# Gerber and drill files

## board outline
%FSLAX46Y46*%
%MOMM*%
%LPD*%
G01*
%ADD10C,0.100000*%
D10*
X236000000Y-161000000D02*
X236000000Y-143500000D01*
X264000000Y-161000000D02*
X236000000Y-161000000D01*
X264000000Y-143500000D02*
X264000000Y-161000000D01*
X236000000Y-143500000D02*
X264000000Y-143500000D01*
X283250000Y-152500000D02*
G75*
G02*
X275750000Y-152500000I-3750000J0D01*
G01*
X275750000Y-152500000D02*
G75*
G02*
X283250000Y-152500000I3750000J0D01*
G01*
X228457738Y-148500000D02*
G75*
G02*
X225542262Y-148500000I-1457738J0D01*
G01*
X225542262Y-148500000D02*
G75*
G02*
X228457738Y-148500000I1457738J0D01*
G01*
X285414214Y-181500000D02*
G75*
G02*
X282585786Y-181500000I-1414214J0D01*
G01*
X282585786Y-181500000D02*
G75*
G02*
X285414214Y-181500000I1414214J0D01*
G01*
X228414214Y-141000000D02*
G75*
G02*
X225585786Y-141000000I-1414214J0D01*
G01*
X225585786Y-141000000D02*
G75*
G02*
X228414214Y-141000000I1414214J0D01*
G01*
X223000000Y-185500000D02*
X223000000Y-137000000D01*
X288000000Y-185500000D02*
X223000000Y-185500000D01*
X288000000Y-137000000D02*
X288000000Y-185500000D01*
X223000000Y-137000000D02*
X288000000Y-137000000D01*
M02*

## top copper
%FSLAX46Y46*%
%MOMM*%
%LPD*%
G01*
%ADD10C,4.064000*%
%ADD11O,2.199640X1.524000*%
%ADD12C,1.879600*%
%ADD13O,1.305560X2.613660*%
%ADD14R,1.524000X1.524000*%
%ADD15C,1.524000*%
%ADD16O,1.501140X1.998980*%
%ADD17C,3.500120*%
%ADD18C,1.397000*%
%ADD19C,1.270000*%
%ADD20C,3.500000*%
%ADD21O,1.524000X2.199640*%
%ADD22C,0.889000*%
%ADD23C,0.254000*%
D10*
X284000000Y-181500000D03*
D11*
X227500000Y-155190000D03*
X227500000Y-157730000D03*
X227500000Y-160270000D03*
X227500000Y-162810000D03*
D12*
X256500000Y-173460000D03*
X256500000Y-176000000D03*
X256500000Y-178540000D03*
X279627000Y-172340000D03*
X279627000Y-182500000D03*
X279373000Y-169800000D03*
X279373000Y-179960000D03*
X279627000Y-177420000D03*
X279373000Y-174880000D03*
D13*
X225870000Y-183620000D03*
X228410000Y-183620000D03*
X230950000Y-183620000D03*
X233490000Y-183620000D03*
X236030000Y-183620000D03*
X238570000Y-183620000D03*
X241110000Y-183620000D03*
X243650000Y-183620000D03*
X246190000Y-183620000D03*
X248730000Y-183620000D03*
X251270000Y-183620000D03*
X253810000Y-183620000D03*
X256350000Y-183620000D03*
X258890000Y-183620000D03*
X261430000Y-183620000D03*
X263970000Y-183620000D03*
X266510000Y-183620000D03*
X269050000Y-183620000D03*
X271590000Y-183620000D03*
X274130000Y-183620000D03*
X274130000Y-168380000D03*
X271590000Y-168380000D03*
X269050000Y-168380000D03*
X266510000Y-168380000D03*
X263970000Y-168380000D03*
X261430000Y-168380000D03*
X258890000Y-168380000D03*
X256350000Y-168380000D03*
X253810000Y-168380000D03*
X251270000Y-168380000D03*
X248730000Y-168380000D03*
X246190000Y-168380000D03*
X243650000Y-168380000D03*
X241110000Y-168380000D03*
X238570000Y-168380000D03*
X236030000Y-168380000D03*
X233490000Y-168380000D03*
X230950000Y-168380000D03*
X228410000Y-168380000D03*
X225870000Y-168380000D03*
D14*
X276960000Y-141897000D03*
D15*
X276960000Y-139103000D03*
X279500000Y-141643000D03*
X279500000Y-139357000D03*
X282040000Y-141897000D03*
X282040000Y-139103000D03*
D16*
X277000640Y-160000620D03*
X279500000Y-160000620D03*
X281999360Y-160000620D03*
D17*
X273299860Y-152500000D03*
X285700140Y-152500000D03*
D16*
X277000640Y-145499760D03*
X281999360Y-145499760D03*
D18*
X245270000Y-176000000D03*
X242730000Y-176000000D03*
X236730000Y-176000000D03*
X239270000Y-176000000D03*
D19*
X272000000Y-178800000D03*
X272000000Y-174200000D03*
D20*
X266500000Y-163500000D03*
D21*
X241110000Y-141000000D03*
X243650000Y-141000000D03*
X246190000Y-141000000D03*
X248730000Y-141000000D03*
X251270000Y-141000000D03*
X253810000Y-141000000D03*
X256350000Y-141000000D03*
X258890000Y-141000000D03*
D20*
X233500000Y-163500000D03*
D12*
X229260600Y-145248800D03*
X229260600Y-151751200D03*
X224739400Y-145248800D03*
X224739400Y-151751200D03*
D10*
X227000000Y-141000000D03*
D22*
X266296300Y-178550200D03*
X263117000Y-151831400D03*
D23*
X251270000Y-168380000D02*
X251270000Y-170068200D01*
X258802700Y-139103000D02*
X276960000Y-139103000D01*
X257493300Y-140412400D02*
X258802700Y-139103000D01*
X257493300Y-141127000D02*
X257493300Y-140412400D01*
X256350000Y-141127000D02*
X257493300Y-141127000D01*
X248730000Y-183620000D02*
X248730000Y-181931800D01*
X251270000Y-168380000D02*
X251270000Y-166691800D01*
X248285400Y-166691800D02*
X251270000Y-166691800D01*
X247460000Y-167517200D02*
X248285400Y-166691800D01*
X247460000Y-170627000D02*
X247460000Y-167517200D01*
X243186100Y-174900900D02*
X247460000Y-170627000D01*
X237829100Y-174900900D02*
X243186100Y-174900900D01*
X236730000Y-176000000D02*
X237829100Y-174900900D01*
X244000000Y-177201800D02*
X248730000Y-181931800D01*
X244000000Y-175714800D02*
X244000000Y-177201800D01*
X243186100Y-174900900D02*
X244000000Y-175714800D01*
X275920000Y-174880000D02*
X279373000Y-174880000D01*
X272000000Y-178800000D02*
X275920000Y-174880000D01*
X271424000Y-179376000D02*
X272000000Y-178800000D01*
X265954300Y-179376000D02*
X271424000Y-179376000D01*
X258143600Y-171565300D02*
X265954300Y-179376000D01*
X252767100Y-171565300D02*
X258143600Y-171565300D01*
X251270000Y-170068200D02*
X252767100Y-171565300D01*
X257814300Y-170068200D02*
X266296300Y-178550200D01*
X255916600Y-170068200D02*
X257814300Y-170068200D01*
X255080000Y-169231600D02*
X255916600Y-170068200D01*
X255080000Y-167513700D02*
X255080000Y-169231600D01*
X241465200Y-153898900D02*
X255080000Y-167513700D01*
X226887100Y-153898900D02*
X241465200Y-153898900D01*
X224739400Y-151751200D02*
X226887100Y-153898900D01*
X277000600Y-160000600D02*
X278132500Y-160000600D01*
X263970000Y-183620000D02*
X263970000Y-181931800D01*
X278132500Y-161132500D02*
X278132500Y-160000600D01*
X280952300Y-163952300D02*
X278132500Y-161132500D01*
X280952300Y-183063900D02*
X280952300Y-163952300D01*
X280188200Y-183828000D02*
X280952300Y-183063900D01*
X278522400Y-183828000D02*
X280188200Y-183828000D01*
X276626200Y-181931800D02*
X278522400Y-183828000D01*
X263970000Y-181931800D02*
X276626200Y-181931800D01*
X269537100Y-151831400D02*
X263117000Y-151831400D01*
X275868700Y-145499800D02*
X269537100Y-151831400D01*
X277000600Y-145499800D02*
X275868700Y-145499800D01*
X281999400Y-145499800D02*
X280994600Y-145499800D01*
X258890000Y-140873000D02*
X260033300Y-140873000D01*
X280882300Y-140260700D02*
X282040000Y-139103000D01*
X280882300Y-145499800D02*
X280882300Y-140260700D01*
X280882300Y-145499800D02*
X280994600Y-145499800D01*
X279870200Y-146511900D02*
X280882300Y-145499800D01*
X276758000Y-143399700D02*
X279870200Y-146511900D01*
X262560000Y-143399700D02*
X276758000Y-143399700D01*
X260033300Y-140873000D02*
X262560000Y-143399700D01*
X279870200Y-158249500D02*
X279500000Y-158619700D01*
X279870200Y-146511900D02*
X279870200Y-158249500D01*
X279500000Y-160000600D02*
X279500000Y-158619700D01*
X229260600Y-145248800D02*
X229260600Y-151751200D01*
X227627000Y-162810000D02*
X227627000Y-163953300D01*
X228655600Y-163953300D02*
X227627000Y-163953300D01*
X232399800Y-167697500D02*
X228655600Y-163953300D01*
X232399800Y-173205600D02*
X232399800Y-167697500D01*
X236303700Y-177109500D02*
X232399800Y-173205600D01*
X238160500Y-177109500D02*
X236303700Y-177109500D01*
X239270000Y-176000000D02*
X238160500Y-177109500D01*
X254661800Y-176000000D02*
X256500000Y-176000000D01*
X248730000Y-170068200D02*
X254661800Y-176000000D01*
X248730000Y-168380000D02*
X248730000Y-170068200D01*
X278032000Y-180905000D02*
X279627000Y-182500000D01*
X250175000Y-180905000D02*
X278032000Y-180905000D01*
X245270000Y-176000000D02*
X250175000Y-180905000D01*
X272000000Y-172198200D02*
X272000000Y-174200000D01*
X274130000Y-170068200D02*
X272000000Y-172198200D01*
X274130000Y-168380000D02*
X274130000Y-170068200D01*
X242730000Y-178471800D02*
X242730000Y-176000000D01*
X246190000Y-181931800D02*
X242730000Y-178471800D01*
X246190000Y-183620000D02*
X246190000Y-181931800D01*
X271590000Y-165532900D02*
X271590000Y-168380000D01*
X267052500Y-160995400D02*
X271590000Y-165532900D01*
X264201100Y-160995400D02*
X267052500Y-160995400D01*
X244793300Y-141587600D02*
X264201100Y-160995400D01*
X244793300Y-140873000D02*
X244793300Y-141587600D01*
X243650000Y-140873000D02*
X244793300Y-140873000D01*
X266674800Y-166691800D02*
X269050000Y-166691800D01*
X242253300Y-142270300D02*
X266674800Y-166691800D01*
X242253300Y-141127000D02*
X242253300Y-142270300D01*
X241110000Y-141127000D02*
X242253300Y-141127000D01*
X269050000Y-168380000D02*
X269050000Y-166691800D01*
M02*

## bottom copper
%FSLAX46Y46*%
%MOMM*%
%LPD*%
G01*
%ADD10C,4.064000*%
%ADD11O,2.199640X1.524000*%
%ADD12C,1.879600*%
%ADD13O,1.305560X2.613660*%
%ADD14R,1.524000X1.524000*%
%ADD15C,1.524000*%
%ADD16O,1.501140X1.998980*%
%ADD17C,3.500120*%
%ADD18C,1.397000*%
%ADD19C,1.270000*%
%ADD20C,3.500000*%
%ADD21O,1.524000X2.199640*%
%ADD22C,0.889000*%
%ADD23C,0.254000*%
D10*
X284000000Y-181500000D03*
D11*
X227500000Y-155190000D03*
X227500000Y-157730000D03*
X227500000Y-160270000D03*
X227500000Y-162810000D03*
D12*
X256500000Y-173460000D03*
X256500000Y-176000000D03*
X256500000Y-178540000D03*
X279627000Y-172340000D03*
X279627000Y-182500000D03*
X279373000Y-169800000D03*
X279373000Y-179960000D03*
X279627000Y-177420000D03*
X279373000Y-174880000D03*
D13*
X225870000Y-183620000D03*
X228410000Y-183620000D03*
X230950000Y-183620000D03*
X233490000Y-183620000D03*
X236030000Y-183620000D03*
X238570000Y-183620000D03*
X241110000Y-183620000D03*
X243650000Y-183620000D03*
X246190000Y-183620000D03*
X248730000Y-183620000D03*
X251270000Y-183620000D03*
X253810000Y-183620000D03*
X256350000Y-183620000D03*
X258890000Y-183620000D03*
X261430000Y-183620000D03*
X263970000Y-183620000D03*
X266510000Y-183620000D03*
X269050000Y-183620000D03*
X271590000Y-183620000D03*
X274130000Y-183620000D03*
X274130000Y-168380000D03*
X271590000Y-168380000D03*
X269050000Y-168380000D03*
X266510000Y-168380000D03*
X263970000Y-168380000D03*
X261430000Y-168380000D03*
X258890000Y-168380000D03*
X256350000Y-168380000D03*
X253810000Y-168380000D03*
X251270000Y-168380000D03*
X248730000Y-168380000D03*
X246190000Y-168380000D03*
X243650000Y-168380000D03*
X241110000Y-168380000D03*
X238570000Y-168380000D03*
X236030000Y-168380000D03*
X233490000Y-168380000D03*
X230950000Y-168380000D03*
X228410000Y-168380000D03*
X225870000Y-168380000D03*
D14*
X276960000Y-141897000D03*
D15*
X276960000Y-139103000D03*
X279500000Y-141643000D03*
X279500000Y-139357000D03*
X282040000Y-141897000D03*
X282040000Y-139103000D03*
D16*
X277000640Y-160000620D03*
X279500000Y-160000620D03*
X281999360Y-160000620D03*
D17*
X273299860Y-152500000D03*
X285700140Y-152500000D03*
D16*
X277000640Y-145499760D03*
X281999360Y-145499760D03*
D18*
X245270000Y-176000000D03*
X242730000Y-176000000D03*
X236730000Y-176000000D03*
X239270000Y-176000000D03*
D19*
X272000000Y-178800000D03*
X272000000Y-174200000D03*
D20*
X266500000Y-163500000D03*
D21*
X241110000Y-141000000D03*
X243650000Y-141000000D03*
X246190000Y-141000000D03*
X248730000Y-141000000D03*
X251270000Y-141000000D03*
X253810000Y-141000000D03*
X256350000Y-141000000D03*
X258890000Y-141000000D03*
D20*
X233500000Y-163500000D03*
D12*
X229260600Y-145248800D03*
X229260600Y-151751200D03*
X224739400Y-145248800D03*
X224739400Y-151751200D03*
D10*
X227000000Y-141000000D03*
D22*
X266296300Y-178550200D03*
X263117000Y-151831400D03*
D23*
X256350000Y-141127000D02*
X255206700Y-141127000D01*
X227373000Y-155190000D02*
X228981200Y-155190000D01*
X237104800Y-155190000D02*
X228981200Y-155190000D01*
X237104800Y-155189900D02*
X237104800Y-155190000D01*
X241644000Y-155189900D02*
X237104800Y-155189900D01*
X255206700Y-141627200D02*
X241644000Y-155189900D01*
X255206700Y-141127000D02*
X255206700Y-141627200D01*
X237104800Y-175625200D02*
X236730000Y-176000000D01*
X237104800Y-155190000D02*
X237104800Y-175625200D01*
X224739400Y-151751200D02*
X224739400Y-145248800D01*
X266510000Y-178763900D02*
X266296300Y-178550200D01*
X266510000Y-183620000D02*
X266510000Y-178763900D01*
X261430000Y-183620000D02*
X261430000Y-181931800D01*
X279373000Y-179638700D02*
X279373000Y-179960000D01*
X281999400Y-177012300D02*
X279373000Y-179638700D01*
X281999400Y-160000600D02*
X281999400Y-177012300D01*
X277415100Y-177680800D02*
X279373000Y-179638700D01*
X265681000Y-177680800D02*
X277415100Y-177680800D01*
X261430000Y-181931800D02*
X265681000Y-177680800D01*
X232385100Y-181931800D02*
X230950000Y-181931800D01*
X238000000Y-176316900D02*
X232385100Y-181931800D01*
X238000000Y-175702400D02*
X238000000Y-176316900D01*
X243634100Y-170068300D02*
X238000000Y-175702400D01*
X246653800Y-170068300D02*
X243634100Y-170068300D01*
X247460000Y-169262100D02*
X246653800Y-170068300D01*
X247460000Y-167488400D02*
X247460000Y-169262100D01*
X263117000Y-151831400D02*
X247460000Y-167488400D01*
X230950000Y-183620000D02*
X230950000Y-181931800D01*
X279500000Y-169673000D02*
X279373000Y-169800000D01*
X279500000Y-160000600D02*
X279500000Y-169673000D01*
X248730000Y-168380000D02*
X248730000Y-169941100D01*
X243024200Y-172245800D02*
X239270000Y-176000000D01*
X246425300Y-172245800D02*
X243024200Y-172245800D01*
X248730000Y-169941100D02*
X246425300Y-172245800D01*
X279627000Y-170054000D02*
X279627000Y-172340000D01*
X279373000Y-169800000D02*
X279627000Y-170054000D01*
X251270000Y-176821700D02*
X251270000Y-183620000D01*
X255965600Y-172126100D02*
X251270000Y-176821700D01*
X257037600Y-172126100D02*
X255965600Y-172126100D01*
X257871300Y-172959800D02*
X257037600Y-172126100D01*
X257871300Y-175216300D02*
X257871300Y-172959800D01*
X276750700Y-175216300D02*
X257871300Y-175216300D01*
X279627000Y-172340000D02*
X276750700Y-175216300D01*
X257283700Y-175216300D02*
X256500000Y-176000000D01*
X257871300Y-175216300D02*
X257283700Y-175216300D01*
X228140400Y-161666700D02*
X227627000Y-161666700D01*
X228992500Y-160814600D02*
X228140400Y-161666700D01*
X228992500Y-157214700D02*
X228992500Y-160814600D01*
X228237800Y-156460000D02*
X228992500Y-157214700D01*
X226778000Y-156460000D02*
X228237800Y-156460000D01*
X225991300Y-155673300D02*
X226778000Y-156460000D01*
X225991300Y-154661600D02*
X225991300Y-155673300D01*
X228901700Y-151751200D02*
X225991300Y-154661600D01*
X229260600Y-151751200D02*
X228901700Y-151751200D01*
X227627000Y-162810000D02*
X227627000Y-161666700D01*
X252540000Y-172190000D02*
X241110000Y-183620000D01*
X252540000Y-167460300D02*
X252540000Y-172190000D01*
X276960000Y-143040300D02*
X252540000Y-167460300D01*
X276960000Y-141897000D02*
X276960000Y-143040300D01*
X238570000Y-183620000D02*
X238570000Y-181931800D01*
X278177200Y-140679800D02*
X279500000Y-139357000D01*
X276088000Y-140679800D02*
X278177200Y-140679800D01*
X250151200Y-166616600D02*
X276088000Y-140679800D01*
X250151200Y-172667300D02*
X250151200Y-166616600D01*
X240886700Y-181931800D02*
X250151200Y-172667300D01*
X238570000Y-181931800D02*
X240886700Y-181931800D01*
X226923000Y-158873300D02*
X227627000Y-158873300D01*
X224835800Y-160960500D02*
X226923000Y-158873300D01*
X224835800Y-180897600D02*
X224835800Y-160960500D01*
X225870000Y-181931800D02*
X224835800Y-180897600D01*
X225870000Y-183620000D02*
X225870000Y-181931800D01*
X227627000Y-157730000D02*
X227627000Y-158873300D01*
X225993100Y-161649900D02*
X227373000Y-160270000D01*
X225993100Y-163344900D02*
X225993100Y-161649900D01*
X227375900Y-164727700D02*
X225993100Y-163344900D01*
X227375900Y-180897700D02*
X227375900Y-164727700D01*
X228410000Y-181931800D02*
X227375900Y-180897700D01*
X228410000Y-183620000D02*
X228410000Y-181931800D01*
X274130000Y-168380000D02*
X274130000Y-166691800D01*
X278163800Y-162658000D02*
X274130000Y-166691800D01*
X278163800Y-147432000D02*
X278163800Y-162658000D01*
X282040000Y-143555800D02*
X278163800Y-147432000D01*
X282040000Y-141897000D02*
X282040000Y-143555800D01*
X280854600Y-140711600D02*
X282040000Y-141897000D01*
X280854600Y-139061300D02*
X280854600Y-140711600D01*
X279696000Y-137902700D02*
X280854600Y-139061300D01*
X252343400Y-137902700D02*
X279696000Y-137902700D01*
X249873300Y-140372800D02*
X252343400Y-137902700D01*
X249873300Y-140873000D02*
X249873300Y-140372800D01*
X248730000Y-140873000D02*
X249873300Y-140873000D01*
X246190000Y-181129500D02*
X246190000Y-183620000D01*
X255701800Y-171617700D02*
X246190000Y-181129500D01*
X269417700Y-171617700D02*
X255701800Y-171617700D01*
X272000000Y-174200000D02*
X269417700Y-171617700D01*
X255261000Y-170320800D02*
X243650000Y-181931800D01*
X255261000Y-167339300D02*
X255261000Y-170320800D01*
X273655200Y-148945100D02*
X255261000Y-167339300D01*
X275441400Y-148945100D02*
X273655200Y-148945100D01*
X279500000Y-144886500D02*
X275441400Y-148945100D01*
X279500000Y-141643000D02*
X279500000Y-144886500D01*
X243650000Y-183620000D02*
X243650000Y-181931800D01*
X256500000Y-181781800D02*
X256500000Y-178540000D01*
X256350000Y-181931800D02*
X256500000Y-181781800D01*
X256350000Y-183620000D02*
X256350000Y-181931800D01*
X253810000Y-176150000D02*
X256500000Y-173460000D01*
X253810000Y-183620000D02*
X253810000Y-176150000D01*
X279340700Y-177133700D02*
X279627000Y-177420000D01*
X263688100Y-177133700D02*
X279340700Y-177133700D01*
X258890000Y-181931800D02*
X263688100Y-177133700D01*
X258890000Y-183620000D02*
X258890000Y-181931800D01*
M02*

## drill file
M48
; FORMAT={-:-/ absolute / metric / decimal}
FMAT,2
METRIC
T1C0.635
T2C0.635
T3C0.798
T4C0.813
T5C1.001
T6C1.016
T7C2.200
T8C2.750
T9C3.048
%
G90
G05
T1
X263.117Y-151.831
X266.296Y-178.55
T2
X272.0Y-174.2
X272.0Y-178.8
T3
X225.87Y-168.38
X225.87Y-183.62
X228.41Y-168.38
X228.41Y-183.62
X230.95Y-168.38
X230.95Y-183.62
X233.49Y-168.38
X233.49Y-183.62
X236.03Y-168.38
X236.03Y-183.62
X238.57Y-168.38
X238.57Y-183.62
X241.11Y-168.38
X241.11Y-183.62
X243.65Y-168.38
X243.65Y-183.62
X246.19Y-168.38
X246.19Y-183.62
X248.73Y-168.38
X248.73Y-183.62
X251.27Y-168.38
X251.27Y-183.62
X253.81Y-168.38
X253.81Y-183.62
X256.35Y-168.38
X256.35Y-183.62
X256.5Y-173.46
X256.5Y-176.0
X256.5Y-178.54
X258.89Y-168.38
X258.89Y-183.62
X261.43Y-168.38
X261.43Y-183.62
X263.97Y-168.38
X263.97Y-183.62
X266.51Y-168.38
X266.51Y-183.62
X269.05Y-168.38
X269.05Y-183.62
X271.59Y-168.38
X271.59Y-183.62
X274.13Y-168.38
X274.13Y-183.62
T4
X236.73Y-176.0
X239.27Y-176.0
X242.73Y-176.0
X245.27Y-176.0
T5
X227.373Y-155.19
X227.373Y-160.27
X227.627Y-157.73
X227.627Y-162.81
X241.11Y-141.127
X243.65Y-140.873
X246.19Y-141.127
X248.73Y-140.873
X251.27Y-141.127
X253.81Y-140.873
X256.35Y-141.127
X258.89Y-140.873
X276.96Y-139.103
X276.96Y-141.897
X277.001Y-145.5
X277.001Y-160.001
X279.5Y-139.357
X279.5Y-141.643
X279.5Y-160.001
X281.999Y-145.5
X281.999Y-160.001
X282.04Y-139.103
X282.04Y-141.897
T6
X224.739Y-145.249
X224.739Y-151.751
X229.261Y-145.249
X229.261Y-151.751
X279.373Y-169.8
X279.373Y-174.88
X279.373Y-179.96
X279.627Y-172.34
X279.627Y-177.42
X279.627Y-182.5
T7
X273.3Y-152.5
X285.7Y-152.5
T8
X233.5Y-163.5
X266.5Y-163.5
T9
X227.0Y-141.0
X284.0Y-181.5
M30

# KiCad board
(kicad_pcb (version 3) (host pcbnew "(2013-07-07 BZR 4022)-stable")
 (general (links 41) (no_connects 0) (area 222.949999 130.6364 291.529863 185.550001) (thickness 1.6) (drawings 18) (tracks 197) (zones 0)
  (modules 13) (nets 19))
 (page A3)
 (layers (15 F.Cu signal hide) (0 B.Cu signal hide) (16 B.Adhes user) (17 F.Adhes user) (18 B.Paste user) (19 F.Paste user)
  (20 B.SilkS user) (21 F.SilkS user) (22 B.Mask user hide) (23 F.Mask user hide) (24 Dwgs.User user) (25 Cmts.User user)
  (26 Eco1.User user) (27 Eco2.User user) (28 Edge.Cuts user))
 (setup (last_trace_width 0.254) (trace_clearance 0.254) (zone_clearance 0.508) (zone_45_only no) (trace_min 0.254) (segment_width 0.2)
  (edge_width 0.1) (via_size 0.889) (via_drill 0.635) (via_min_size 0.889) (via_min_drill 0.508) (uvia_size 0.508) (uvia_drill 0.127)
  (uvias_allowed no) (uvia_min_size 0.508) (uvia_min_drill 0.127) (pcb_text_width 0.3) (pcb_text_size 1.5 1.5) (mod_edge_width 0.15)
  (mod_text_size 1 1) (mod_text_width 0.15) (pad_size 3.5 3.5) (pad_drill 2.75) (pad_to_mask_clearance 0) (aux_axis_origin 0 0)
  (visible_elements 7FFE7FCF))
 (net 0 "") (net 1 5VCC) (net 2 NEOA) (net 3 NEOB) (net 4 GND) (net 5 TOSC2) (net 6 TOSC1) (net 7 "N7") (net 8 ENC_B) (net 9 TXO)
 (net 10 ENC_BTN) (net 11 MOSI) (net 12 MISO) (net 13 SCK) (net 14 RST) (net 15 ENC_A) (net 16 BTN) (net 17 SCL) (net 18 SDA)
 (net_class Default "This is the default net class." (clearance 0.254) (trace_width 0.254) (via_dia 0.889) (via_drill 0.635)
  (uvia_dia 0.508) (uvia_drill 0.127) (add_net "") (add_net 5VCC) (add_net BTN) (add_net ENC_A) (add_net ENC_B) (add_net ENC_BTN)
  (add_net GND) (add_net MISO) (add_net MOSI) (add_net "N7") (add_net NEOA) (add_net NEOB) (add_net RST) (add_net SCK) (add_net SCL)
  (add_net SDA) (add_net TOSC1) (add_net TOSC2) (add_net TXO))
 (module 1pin (layer F.Cu) (at 284 181.5)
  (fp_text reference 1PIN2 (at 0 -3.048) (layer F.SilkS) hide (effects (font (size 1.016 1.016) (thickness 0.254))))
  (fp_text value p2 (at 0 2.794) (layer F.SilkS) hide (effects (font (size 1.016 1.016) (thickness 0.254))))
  (pad 1 thru_hole circle (at 0 0) (size 4.064 4.064) (drill 3.048) (layers *.Cu *.Mask F.SilkS)))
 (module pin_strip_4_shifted (layer F.Cu) (at 227.5 159 270)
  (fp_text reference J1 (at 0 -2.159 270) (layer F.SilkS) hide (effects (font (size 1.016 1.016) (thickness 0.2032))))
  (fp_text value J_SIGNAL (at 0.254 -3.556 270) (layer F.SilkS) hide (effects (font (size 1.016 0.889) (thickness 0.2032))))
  (pad 1 thru_hole oval (at -3.81 0.127 270) (size 1.524 2.19964) (drill 1.00076 (offset 0 -0.127)) (layers *.Cu *.Mask F.SilkS)
   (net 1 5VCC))
  (pad 2 thru_hole oval (at -1.27 -0.127 270) (size 1.524 2.19964) (drill 1.00076 (offset 0 0.127)) (layers *.Cu *.Mask F.SilkS)
   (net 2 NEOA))
  (pad 3 thru_hole oval (at 1.27 0.127 270) (size 1.524 2.19964) (drill 1.00076 (offset 0 -0.127)) (layers *.Cu *.Mask F.SilkS) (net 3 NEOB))
  (pad 4 thru_hole oval (at 3.81 -0.127 270) (size 1.524 2.19964) (drill 1.00076 (offset 0 0.127)) (layers *.Cu *.Mask F.SilkS) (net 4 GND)))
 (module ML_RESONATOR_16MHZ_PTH (layer F.Cu) (at 256.5 176 270)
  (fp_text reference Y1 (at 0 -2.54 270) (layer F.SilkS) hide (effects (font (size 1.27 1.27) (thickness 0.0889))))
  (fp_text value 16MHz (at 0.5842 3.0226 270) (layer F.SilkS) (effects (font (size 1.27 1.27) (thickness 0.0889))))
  (pad 1 thru_hole circle (at -2.54 0 270) (size 1.8796 1.8796) (drill 0.79756) (layers *.Cu *.Mask F.Paste F.SilkS) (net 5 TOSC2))
  (pad 2 thru_hole circle (at 0 0 270) (size 1.8796 1.8796) (drill 0.79756) (layers *.Cu *.Mask F.Paste F.SilkS) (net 4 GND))
  (pad 3 thru_hole circle (at 2.54 0 270) (size 1.8796 1.8796) (drill 0.79756) (layers *.Cu *.Mask F.Paste F.SilkS) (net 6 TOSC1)))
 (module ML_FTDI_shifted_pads (layer F.Cu) (at 279.5 182.5 90)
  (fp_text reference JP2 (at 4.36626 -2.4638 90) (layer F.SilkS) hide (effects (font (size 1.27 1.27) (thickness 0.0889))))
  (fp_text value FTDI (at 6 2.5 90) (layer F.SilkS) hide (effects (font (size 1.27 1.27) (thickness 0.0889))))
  (pad CTS thru_hole circle (at 10.16 0.127 90) (size 1.8796 1.8796) (drill 1.016) (layers *.Cu *.Mask F.Paste F.SilkS) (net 4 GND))
  (pad DTR thru_hole circle (at 0 0.127 90) (size 1.8796 1.8796) (drill 1.016) (layers *.Cu *.Mask F.Paste F.SilkS) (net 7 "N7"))
  (pad GND thru_hole circle (at 12.7 -0.127 90) (size 1.8796 1.8796) (drill 1.016) (layers *.Cu *.Mask F.Paste F.SilkS) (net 4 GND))
  (pad RXI thru_hole circle (at 2.54 -0.127 90) (size 1.8796 1.8796) (drill 1.016) (layers *.Cu *.Mask F.Paste F.SilkS) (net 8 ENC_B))
  (pad TXO thru_hole circle (at 5.08 0.127 90) (size 1.8796 1.8796) (drill 1.016) (layers *.Cu *.Mask F.Paste F.SilkS) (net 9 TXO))
  (pad VCC thru_hole circle (at 7.62 -0.127 90) (size 1.8796 1.8796) (drill 1.016) (layers *.Cu *.Mask F.Paste F.SilkS) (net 1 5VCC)))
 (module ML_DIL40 (layer F.Cu) (at 250 176)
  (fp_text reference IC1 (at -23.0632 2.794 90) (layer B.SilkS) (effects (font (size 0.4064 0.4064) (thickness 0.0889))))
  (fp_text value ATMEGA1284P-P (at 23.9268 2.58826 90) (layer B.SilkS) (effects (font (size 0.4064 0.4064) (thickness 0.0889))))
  (pad 1 thru_hole oval (at -24.13 7.62) (size 1.30556 2.61366) (drill 0.79756) (layers *.Cu *.Mask F.Paste F.SilkS) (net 2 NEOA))
  (pad 2 thru_hole oval (at -21.59 7.62) (size 1.30556 2.61366) (drill 0.79756) (layers *.Cu *.Mask F.Paste F.SilkS) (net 3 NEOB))
  (pad 3 thru_hole oval (at -19.05 7.62) (size 1.30556 2.61366) (drill 0.79756) (layers *.Cu *.Mask F.Paste F.SilkS) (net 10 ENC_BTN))
  (pad 4 thru_hole oval (at -16.51 7.62) (size 1.30556 2.61366) (drill 0.79756) (layers *.Cu *.Mask F.Paste F.SilkS))
  (pad 5 thru_hole oval (at -13.97 7.62) (size 1.30556 2.61366) (drill 0.79756) (layers *.Cu *.Mask F.Paste F.SilkS))
  (pad 6 thru_hole oval (at -11.43 7.62) (size 1.30556 2.61366) (drill 0.79756) (layers *.Cu *.Mask F.Paste F.SilkS) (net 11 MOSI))
  (pad 7 thru_hole oval (at -8.89 7.62) (size 1.30556 2.61366) (drill 0.79756) (layers *.Cu *.Mask F.Paste F.SilkS) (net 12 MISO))
  (pad 8 thru_hole oval (at -6.35 7.62) (size 1.30556 2.61366) (drill 0.79756) (layers *.Cu *.Mask F.Paste F.SilkS) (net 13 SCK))
  (pad 9 thru_hole oval (at -3.81 7.62) (size 1.30556 2.61366) (drill 0.79756) (layers *.Cu *.Mask F.Paste F.SilkS) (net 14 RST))
  (pad 10 thru_hole oval (at -1.27 7.62) (size 1.30556 2.61366) (drill 0.79756) (layers *.Cu *.Mask F.Paste F.SilkS) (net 1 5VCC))
  (pad 11 thru_hole oval (at 1.27 7.62) (size 1.30556 2.61366) (drill 0.79756) (layers *.Cu *.Mask F.Paste F.SilkS) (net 4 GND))
  (pad 12 thru_hole oval (at 3.81 7.62) (size 1.30556 2.61366) (drill 0.79756) (layers *.Cu *.Mask F.Paste F.SilkS) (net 5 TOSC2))
  (pad 13 thru_hole oval (at 6.35 7.62) (size 1.30556 2.61366) (drill 0.79756) (layers *.Cu *.Mask F.Paste F.SilkS) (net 6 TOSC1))
  (pad 14 thru_hole oval (at 8.89 7.62) (size 1.30556 2.61366) (drill 0.79756) (layers *.Cu *.Mask F.Paste F.SilkS) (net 9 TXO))
  (pad 15 thru_hole oval (at 11.43 7.62) (size 1.30556 2.61366) (drill 0.79756) (layers *.Cu *.Mask F.Paste F.SilkS) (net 8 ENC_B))
  (pad 16 thru_hole oval (at 13.97 7.62) (size 1.30556 2.61366) (drill 0.79756) (layers *.Cu *.Mask F.Paste F.SilkS) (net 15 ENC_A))
  (pad 17 thru_hole oval (at 16.51 7.62) (size 1.30556 2.61366) (drill 0.79756) (layers *.Cu *.Mask F.Paste F.SilkS) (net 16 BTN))
  (pad 18 thru_hole oval (at 19.05 7.62) (size 1.30556 2.61366) (drill 0.79756) (layers *.Cu *.Mask F.Paste F.SilkS))
  (pad 19 thru_hole oval (at 21.59 7.62) (size 1.30556 2.61366) (drill 0.79756) (layers *.Cu *.Mask F.Paste F.SilkS))
  (pad 20 thru_hole oval (at 24.13 7.62) (size 1.30556 2.61366) (drill 0.79756) (layers *.Cu *.Mask F.Paste F.SilkS))
  (pad 21 thru_hole oval (at 24.13 -7.62) (size 1.30556 2.61366) (drill 0.79756) (layers *.Cu *.Mask F.Paste F.SilkS) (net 14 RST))
  (pad 22 thru_hole oval (at 21.59 -7.62) (size 1.30556 2.61366) (drill 0.79756) (layers *.Cu *.Mask F.Paste F.SilkS) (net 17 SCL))
  (pad 23 thru_hole oval (at 19.05 -7.62) (size 1.30556 2.61366) (drill 0.79756) (layers *.Cu *.Mask F.Paste F.SilkS) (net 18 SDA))
  (pad 24 thru_hole oval (at 16.51 -7.62) (size 1.30556 2.61366) (drill 0.79756) (layers *.Cu *.Mask F.Paste F.SilkS))
  (pad 25 thru_hole oval (at 13.97 -7.62) (size 1.30556 2.61366) (drill 0.79756) (layers *.Cu *.Mask F.Paste F.SilkS))
  (pad 26 thru_hole oval (at 11.43 -7.62) (size 1.30556 2.61366) (drill 0.79756) (layers *.Cu *.Mask F.Paste F.SilkS))
  (pad 27 thru_hole oval (at 8.89 -7.62) (size 1.30556 2.61366) (drill 0.79756) (layers *.Cu *.Mask F.Paste F.SilkS))
  (pad 28 thru_hole oval (at 6.35 -7.62) (size 1.30556 2.61366) (drill 0.79756) (layers *.Cu *.Mask F.Paste F.SilkS))
  (pad 29 thru_hole oval (at 3.81 -7.62) (size 1.30556 2.61366) (drill 0.79756) (layers *.Cu *.Mask F.Paste F.SilkS))
  (pad 30 thru_hole oval (at 1.27 -7.62) (size 1.30556 2.61366) (drill 0.79756) (layers *.Cu *.Mask F.Paste F.SilkS) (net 1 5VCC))
  (pad 31 thru_hole oval (at -1.27 -7.62) (size 1.30556 2.61366) (drill 0.79756) (layers *.Cu *.Mask F.Paste F.SilkS) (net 4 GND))
  (pad 32 thru_hole oval (at -3.81 -7.62) (size 1.30556 2.61366) (drill 0.79756) (layers *.Cu *.Mask F.Paste F.SilkS))
  (pad 33 thru_hole oval (at -6.35 -7.62) (size 1.30556 2.61366) (drill 0.79756) (layers *.Cu *.Mask F.Paste F.SilkS))
  (pad 34 thru_hole oval (at -8.89 -7.62) (size 1.30556 2.61366) (drill 0.79756) (layers *.Cu *.Mask F.Paste F.SilkS))
  (pad 35 thru_hole oval (at -11.43 -7.62) (size 1.30556 2.61366) (drill 0.79756) (layers *.Cu *.Mask F.Paste F.SilkS))
  (pad 36 thru_hole oval (at -13.97 -7.62) (size 1.30556 2.61366) (drill 0.79756) (layers *.Cu *.Mask F.Paste F.SilkS))
  (pad 37 thru_hole oval (at -16.51 -7.62) (size 1.30556 2.61366) (drill 0.79756) (layers *.Cu *.Mask F.Paste F.SilkS))
  (pad 38 thru_hole oval (at -19.05 -7.62) (size 1.30556 2.61366) (drill 0.79756) (layers *.Cu *.Mask F.Paste F.SilkS))
  (pad 39 thru_hole oval (at -21.59 -7.62) (size 1.30556 2.61366) (drill 0.79756) (layers *.Cu *.Mask F.Paste F.SilkS))
  (pad 40 thru_hole oval (at -24.13 -7.62) (size 1.30556 2.61366) (drill 0.79756) (layers *.Cu *.Mask F.Paste F.SilkS)))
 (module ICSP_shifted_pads (layer F.Cu) (at 279.5 140.5)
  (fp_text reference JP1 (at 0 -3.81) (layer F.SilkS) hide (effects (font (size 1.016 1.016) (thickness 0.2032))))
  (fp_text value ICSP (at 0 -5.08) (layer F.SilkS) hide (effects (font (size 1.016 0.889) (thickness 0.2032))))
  (pad 1 thru_hole rect (at -2.54 1.397) (size 1.524 1.524) (drill 1.00076) (layers *.Cu *.Mask F.SilkS) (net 12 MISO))
  (pad 2 thru_hole circle (at -2.54 -1.397) (size 1.524 1.524) (drill 1.00076) (layers *.Cu *.Mask F.SilkS) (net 1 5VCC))
  (pad 3 thru_hole circle (at 0 1.143) (size 1.524 1.524) (drill 1.00076) (layers *.Cu *.Mask F.SilkS) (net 13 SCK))
  (pad 4 thru_hole circle (at 0 -1.143) (size 1.524 1.524) (drill 1.00076) (layers *.Cu *.Mask F.SilkS) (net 11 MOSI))
  (pad 5 thru_hole circle (at 2.54 1.397) (size 1.524 1.524) (drill 1.00076) (layers *.Cu *.Mask F.SilkS) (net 14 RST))
  (pad 6 thru_hole circle (at 2.54 -1.397) (size 1.524 1.524) (drill 1.00076) (layers *.Cu *.Mask F.SilkS) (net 4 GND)))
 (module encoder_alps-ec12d (layer F.Cu) (at 279.5 152.5) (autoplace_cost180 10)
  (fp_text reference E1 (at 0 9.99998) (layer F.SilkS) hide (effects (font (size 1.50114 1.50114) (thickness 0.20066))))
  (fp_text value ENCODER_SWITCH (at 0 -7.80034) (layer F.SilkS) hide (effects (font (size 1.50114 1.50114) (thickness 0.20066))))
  (pad 1 thru_hole oval (at -2.49936 7.50062) (size 1.50114 1.99898) (drill 1.00076) (layers *.Cu *.Mask F.SilkS) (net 15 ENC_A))
  (pad 2 thru_hole oval (at 0 7.50062) (size 1.50114 1.99898) (drill 1.00076) (layers *.Cu *.Mask F.SilkS) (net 4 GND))
  (pad 3 thru_hole oval (at 2.49936 7.50062) (size 1.50114 1.99898) (drill 1.00076) (layers *.Cu *.Mask F.SilkS) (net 8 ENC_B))
  (pad "" thru_hole circle (at -6.20014 0) (size 3.50012 3.50012) (drill 2.19964) (layers *.Cu *.Mask F.SilkS))
  (pad "" thru_hole circle (at 6.20014 0) (size 3.50012 3.50012) (drill 2.19964) (layers *.Cu *.Mask F.SilkS))
  (pad 5 thru_hole oval (at -2.49936 -7.00024) (size 1.50114 1.99898) (drill 1.00076) (layers *.Cu *.Mask F.SilkS) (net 10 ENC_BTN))
  (pad 4 thru_hole oval (at 2.49936 -7.00024) (size 1.50114 1.99898) (drill 1.00076) (layers *.Cu *.Mask F.SilkS) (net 4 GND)))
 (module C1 (layer F.Cu) (at 244 176 180)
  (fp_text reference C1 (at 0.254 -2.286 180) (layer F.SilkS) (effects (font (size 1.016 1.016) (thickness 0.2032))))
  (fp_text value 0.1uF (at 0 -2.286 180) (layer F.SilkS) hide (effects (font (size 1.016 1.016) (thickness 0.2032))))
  (pad 1 thru_hole circle (at -1.27 0 180) (size 1.397 1.397) (drill 0.8128) (layers *.Cu *.Mask F.SilkS) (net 7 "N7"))
  (pad 2 thru_hole circle (at 1.27 0 180) (size 1.397 1.397) (drill 0.8128) (layers *.Cu *.Mask F.SilkS) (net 14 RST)))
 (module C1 (layer F.Cu) (at 238 176)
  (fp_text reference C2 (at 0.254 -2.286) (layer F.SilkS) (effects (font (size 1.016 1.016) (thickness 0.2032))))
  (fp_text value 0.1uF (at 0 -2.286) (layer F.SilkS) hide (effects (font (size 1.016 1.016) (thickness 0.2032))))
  (pad 1 thru_hole circle (at -1.27 0) (size 1.397 1.397) (drill 0.8128) (layers *.Cu *.Mask F.SilkS) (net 1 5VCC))
  (pad 2 thru_hole circle (at 1.27 0) (size 1.397 1.397) (drill 0.8128) (layers *.Cu *.Mask F.SilkS) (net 4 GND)))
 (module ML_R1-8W (layer F.Cu) (at 272 176.5 90)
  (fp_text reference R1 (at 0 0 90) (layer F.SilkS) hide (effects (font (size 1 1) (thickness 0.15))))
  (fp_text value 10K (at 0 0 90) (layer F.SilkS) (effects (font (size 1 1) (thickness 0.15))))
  (pad 1 thru_hole circle (at -2.3 0 90) (size 1.27 1.27) (drill 0.635) (layers *.Cu *.Mask F.SilkS) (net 1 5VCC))
  (pad 2 thru_hole circle (at 2.3 0 90) (size 1.27 1.27) (drill 0.635) (layers *.Cu *.Mask F.SilkS) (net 14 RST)))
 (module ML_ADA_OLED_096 (layer F.Cu) (at 250 141)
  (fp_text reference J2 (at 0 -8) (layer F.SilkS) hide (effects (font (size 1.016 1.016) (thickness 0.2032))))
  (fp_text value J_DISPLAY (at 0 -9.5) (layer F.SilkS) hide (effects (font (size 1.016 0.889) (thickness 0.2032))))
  (pad 9 thru_hole circle (at 16.5 22.5) (size 3.5 3.5) (drill 2.75) (layers *.Cu *.Mask F.SilkS))
  (pad 1 thru_hole oval (at -8.89 0.127) (size 1.524 2.19964) (drill 1.00076 (offset 0 -0.127)) (layers *.Cu *.Mask F.SilkS) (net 18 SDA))
  (pad 2 thru_hole oval (at -6.35 -0.127) (size 1.524 2.19964) (drill 1.00076 (offset 0 0.127)) (layers *.Cu *.Mask F.SilkS) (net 17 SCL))
  (pad 3 thru_hole oval (at -3.81 0.127) (size 1.524 2.19964) (drill 1.00076 (offset 0 -0.127)) (layers *.Cu *.Mask F.SilkS))
  (pad 4 thru_hole oval (at -1.27 -0.127) (size 1.524 2.19964) (drill 1.00076 (offset 0 0.127)) (layers *.Cu *.Mask F.SilkS) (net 14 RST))
  (pad 5 thru_hole oval (at 1.27 0.127) (size 1.524 2.19964) (drill 1.00076 (offset 0 -0.127)) (layers *.Cu *.Mask F.SilkS))
  (pad 6 thru_hole oval (at 3.81 -0.127) (size 1.524 2.19964) (drill 1.00076 (offset 0 0.127)) (layers *.Cu *.Mask F.SilkS))
  (pad 7 thru_hole oval (at 6.35 0.127) (size 1.524 2.19964) (drill 1.00076 (offset 0 -0.127)) (layers *.Cu *.Mask F.SilkS) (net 1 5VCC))
  (pad 8 thru_hole oval (at 8.89 -0.127) (size 1.524 2.19964) (drill 1.00076 (offset 0 0.127)) (layers *.Cu *.Mask F.SilkS) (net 4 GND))
  (pad 9 thru_hole circle (at -16.5 22.5) (size 3.5 3.5) (drill 2.75) (layers *.Cu *.Mask F.SilkS)))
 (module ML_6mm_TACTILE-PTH (layer F.Cu) (at 227 148.5 270)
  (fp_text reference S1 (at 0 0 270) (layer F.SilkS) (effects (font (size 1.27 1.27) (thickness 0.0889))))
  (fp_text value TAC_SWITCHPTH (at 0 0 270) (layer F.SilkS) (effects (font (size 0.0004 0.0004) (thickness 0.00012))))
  (pad 1 thru_hole circle (at -3.2512 -2.2606 270) (size 1.8796 1.8796) (drill 1.016) (layers *.Cu *.Mask F.Paste F.SilkS) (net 4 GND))
  (pad 2 thru_hole circle (at 3.2512 -2.2606 270) (size 1.8796 1.8796) (drill 1.016) (layers *.Cu *.Mask F.Paste F.SilkS) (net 4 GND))
  (pad 3 thru_hole circle (at -3.2512 2.2606 270) (size 1.8796 1.8796) (drill 1.016) (layers *.Cu *.Mask F.Paste F.SilkS) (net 16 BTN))
  (pad 4 thru_hole circle (at 3.2512 2.2606 270) (size 1.8796 1.8796) (drill 1.016) (layers *.Cu *.Mask F.Paste F.SilkS) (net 16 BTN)))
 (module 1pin (layer F.Cu) (at 227 141)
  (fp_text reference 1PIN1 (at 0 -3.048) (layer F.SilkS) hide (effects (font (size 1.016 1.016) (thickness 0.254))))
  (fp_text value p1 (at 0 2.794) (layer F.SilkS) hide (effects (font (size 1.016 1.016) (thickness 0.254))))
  (pad 1 thru_hole circle (at 0 0) (size 4.064 4.064) (drill 3.048) (layers *.Cu *.Mask F.SilkS)))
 (gr_line (start 236 161) (end 236 143.5) (angle 90) (layer Edge.Cuts) (width 0.1))
 (gr_line (start 264 161) (end 236 161) (angle 90) (layer Edge.Cuts) (width 0.1))
 (gr_line (start 264 143.5) (end 264 161) (angle 90) (layer Edge.Cuts) (width 0.1))
 (gr_line (start 236 143.5) (end 264 143.5) (angle 90) (layer Edge.Cuts) (width 0.1))
 (gr_circle (center 279.5 152.5) (end 282.5 154.75) (layer Edge.Cuts) (width 0.1))
 (gr_circle (center 227 148.5) (end 228.25 149.25) (layer Edge.Cuts) (width 0.1))
 (gr_circle (center 284 181.5) (end 285 182.5) (layer Edge.Cuts) (width 0.1))
 (gr_circle (center 227 141) (end 228 142) (layer Edge.Cuts) (width 0.1))
 (gr_line (start 223 185.5) (end 223 137) (angle 90) (layer Edge.Cuts) (width 0.1))
 (gr_line (start 288 185.5) (end 223 185.5) (angle 90) (layer Edge.Cuts) (width 0.1))
 (gr_line (start 288 137) (end 288 185.5) (angle 90) (layer Edge.Cuts) (width 0.1))
 (gr_line (start 223 137) (end 288 137) (angle 90) (layer Edge.Cuts) (width 0.1))
 (segment (start 256.35 141.127) (end 255.2067 141.127) (width 0.254) (layer B.Cu) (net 1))
 (segment (start 227.373 155.19) (end 228.9812 155.19) (width 0.254) (layer B.Cu) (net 1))
 (segment (start 237.1048 155.19) (end 228.9812 155.19) (width 0.254) (layer B.Cu) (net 1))
 (segment (start 237.1048 155.1899) (end 237.1048 155.19) (width 0.254) (layer B.Cu) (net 1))
 (segment (start 241.644 155.1899) (end 237.1048 155.1899) (width 0.254) (layer B.Cu) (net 1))
 (segment (start 255.2067 141.6272) (end 241.644 155.1899) (width 0.254) (layer B.Cu) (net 1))
 (segment (start 255.2067 141.127) (end 255.2067 141.6272) (width 0.254) (layer B.Cu) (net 1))
 (segment (start 237.1048 175.6252) (end 236.73 176) (width 0.254) (layer B.Cu) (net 1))
 (segment (start 237.1048 155.19) (end 237.1048 175.6252) (width 0.254) (layer B.Cu) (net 1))
 (segment (start 251.27 168.38) (end 251.27 170.0682) (width 0.254) (layer F.Cu) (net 1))
 (segment (start 258.8027 139.103) (end 276.96 139.103) (width 0.254) (layer F.Cu) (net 1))
 (segment (start 257.4933 140.4124) (end 258.8027 139.103) (width 0.254) (layer F.Cu) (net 1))
 (segment (start 257.4933 141.127) (end 257.4933 140.4124) (width 0.254) (layer F.Cu) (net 1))
 (segment (start 256.35 141.127) (end 257.4933 141.127) (width 0.254) (layer F.Cu) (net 1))
 (segment (start 248.73 183.62) (end 248.73 181.9318) (width 0.254) (layer F.Cu) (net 1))
 (segment (start 251.27 168.38) (end 251.27 166.6918) (width 0.254) (layer F.Cu) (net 1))
 (segment (start 248.2854 166.6918) (end 251.27 166.6918) (width 0.254) (layer F.Cu) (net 1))
 (segment (start 247.46 167.5172) (end 248.2854 166.6918) (width 0.254) (layer F.Cu) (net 1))
 (segment (start 247.46 170.627) (end 247.46 167.5172) (width 0.254) (layer F.Cu) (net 1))
 (segment (start 243.1861 174.9009) (end 247.46 170.627) (width 0.254) (layer F.Cu) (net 1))
 (segment (start 237.8291 174.9009) (end 243.1861 174.9009) (width 0.254) (layer F.Cu) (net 1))
 (segment (start 236.73 176) (end 237.8291 174.9009) (width 0.254) (layer F.Cu) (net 1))
 (segment (start 244 177.2018) (end 248.73 181.9318) (width 0.254) (layer F.Cu) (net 1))
 (segment (start 244 175.7148) (end 244 177.2018) (width 0.254) (layer F.Cu) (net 1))
 (segment (start 243.1861 174.9009) (end 244 175.7148) (width 0.254) (layer F.Cu) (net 1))
 (segment (start 275.92 174.88) (end 279.373 174.88) (width 0.254) (layer F.Cu) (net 1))
 (segment (start 272 178.8) (end 275.92 174.88) (width 0.254) (layer F.Cu) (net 1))
 (segment (start 271.424 179.376) (end 272 178.8) (width 0.254) (layer F.Cu) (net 1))
 (segment (start 265.9543 179.376) (end 271.424 179.376) (width 0.254) (layer F.Cu) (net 1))
 (segment (start 258.1436 171.5653) (end 265.9543 179.376) (width 0.254) (layer F.Cu) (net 1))
 (segment (start 252.7671 171.5653) (end 258.1436 171.5653) (width 0.254) (layer F.Cu) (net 1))
 (segment (start 251.27 170.0682) (end 252.7671 171.5653) (width 0.254) (layer F.Cu) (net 1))
 (via (at 266.2963 178.5502) (size 0.889) (layers F.Cu B.Cu) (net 16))
 (segment (start 224.7394 151.7512) (end 224.7394 145.2488) (width 0.254) (layer B.Cu) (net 16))
 (segment (start 266.51 178.7639) (end 266.2963 178.5502) (width 0.254) (layer B.Cu) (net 16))
 (segment (start 266.51 183.62) (end 266.51 178.7639) (width 0.254) (layer B.Cu) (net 16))
 (segment (start 257.8143 170.0682) (end 266.2963 178.5502) (width 0.254) (layer F.Cu) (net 16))
 (segment (start 255.9166 170.0682) (end 257.8143 170.0682) (width 0.254) (layer F.Cu) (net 16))
 (segment (start 255.08 169.2316) (end 255.9166 170.0682) (width 0.254) (layer F.Cu) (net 16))
 (segment (start 255.08 167.5137) (end 255.08 169.2316) (width 0.254) (layer F.Cu) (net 16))
 (segment (start 241.4652 153.8989) (end 255.08 167.5137) (width 0.254) (layer F.Cu) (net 16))
 (segment (start 226.8871 153.8989) (end 241.4652 153.8989) (width 0.254) (layer F.Cu) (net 16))
 (segment (start 224.7394 151.7512) (end 226.8871 153.8989) (width 0.254) (layer F.Cu) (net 16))
 (segment (start 277.0006 160.0006) (end 278.1325 160.0006) (width 0.254) (layer F.Cu) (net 15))
 (segment (start 263.97 183.62) (end 263.97 181.9318) (width 0.254) (layer F.Cu) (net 15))
 (segment (start 278.1325 161.1325) (end 278.1325 160.0006) (width 0.254) (layer F.Cu) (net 15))
 (segment (start 280.9523 163.9523) (end 278.1325 161.1325) (width 0.254) (layer F.Cu) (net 15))
 (segment (start 280.9523 183.0639) (end 280.9523 163.9523) (width 0.254) (layer F.Cu) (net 15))
 (segment (start 280.1882 183.828) (end 280.9523 183.0639) (width 0.254) (layer F.Cu) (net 15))
 (segment (start 278.5224 183.828) (end 280.1882 183.828) (width 0.254) (layer F.Cu) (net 15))
 (segment (start 276.6262 181.9318) (end 278.5224 183.828) (width 0.254) (layer F.Cu) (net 15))
 (segment (start 263.97 181.9318) (end 276.6262 181.9318) (width 0.254) (layer F.Cu) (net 15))
 (segment (start 261.43 183.62) (end 261.43 181.9318) (width 0.254) (layer B.Cu) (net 8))
 (segment (start 279.373 179.6387) (end 279.373 179.96) (width 0.254) (layer B.Cu) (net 8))
 (segment (start 281.9994 177.0123) (end 279.373 179.6387) (width 0.254) (layer B.Cu) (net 8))
 (segment (start 281.9994 160.0006) (end 281.9994 177.0123) (width 0.254) (layer B.Cu) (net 8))
 (segment (start 277.4151 177.6808) (end 279.373 179.6387) (width 0.254) (layer B.Cu) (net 8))
 (segment (start 265.681 177.6808) (end 277.4151 177.6808) (width 0.254) (layer B.Cu) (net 8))
 (segment (start 261.43 181.9318) (end 265.681 177.6808) (width 0.254) (layer B.Cu) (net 8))
 (via (at 263.117 151.8314) (size 0.889) (layers F.Cu B.Cu) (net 10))
 (segment (start 232.3851 181.9318) (end 230.95 181.9318) (width 0.254) (layer B.Cu) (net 10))
 (segment (start 238 176.3169) (end 232.3851 181.9318) (width 0.254) (layer B.Cu) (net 10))
 (segment (start 238 175.7024) (end 238 176.3169) (width 0.254) (layer B.Cu) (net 10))
 (segment (start 243.6341 170.0683) (end 238 175.7024) (width 0.254) (layer B.Cu) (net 10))
 (segment (start 246.6538 170.0683) (end 243.6341 170.0683) (width 0.254) (layer B.Cu) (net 10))
 (segment (start 247.46 169.2621) (end 246.6538 170.0683) (width 0.254) (layer B.Cu) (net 10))
 (segment (start 247.46 167.4884) (end 247.46 169.2621) (width 0.254) (layer B.Cu) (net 10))
 (segment (start 263.117 151.8314) (end 247.46 167.4884) (width 0.254) (layer B.Cu) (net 10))
 (segment (start 269.5371 151.8314) (end 263.117 151.8314) (width 0.254) (layer F.Cu) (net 10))
 (segment (start 275.8687 145.4998) (end 269.5371 151.8314) (width 0.254) (layer F.Cu) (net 10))
 (segment (start 230.95 183.62) (end 230.95 181.9318) (width 0.254) (layer B.Cu) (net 10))
 (segment (start 277.0006 145.4998) (end 275.8687 145.4998) (width 0.254) (layer F.Cu) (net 10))
 (segment (start 281.9994 145.4998) (end 280.9946 145.4998) (width 0.254) (layer F.Cu) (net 4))
 (segment (start 258.89 140.873) (end 260.0333 140.873) (width 0.254) (layer F.Cu) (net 4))
 (segment (start 280.8823 140.2607) (end 282.04 139.103) (width 0.254) (layer F.Cu) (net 4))
 (segment (start 280.8823 145.4998) (end 280.8823 140.2607) (width 0.254) (layer F.Cu) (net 4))
 (segment (start 280.8823 145.4998) (end 280.9946 145.4998) (width 0.254) (layer F.Cu) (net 4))
 (segment (start 279.8702 146.5119) (end 280.8823 145.4998) (width 0.254) (layer F.Cu) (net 4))
 (segment (start 276.758 143.3997) (end 279.8702 146.5119) (width 0.254) (layer F.Cu) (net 4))
 (segment (start 262.56 143.3997) (end 276.758 143.3997) (width 0.254) (layer F.Cu) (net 4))
 (segment (start 260.0333 140.873) (end 262.56 143.3997) (width 0.254) (layer F.Cu) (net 4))
 (segment (start 279.8702 158.2495) (end 279.5 158.6197) (width 0.254) (layer F.Cu) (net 4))
 (segment (start 279.8702 146.5119) (end 279.8702 158.2495) (width 0.254) (layer F.Cu) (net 4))
 (segment (start 279.5 160.0006) (end 279.5 158.6197) (width 0.254) (layer F.Cu) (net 4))
 (segment (start 279.5 169.673) (end 279.373 169.8) (width 0.254) (layer B.Cu) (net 4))
 (segment (start 279.5 160.0006) (end 279.5 169.673) (width 0.254) (layer B.Cu) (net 4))
 (segment (start 229.2606 145.2488) (end 229.2606 151.7512) (width 0.254) (layer F.Cu) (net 4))
 (segment (start 227.627 162.81) (end 227.627 163.9533) (width 0.254) (layer F.Cu) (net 4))
 (segment (start 228.6556 163.9533) (end 227.627 163.9533) (width 0.254) (layer F.Cu) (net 4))
 (segment (start 232.3998 167.6975) (end 228.6556 163.9533) (width 0.254) (layer F.Cu) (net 4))
 (segment (start 232.3998 173.2056) (end 232.3998 167.6975) (width 0.254) (layer F.Cu) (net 4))
 (segment (start 236.3037 177.1095) (end 232.3998 173.2056) (width 0.254) (layer F.Cu) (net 4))
 (segment (start 238.1605 177.1095) (end 236.3037 177.1095) (width 0.254) (layer F.Cu) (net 4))
 (segment (start 239.27 176) (end 238.1605 177.1095) (width 0.254) (layer F.Cu) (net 4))
 (segment (start 248.73 168.38) (end 248.73 169.9411) (width 0.254) (layer B.Cu) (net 4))
 (segment (start 243.0242 172.2458) (end 239.27 176) (width 0.254) (layer B.Cu) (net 4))
 (segment (start 246.4253 172.2458) (end 243.0242 172.2458) (width 0.254) (layer B.Cu) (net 4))
 (segment (start 248.73 169.9411) (end 246.4253 172.2458) (width 0.254) (layer B.Cu) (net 4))
 (segment (start 254.6618 176) (end 256.5 176) (width 0.254) (layer F.Cu) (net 4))
 (segment (start 248.73 170.0682) (end 254.6618 176) (width 0.254) (layer F.Cu) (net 4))
 (segment (start 248.73 168.38) (end 248.73 170.0682) (width 0.254) (layer F.Cu) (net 4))
 (segment (start 279.627 170.054) (end 279.627 172.34) (width 0.254) (layer B.Cu) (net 4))
 (segment (start 279.373 169.8) (end 279.627 170.054) (width 0.254) (layer B.Cu) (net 4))
 (segment (start 251.27 176.8217) (end 251.27 183.62) (width 0.254) (layer B.Cu) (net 4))
 (segment (start 255.9656 172.1261) (end 251.27 176.8217) (width 0.254) (layer B.Cu) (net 4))
 (segment (start 257.0376 172.1261) (end 255.9656 172.1261) (width 0.254) (layer B.Cu) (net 4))
 (segment (start 257.8713 172.9598) (end 257.0376 172.1261) (width 0.254) (layer B.Cu) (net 4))
 (segment (start 257.8713 175.2163) (end 257.8713 172.9598) (width 0.254) (layer B.Cu) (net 4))
 (segment (start 276.7507 175.2163) (end 257.8713 175.2163) (width 0.254) (layer B.Cu) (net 4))
 (segment (start 279.627 172.34) (end 276.7507 175.2163) (width 0.254) (layer B.Cu) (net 4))
 (segment (start 257.2837 175.2163) (end 256.5 176) (width 0.254) (layer B.Cu) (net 4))
 (segment (start 257.8713 175.2163) (end 257.2837 175.2163) (width 0.254) (layer B.Cu) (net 4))
 (segment (start 228.1404 161.6667) (end 227.627 161.6667) (width 0.254) (layer B.Cu) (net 4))
 (segment (start 228.9925 160.8146) (end 228.1404 161.6667) (width 0.254) (layer B.Cu) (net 4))
 (segment (start 228.9925 157.2147) (end 228.9925 160.8146) (width 0.254) (layer B.Cu) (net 4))
 (segment (start 228.2378 156.46) (end 228.9925 157.2147) (width 0.254) (layer B.Cu) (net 4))
 (segment (start 226.778 156.46) (end 228.2378 156.46) (width 0.254) (layer B.Cu) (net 4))
 (segment (start 225.9913 155.6733) (end 226.778 156.46) (width 0.254) (layer B.Cu) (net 4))
 (segment (start 225.9913 154.6616) (end 225.9913 155.6733) (width 0.254) (layer B.Cu) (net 4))
 (segment (start 228.9017 151.7512) (end 225.9913 154.6616) (width 0.254) (layer B.Cu) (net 4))
 (segment (start 229.2606 151.7512) (end 228.9017 151.7512) (width 0.254) (layer B.Cu) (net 4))
 (segment (start 227.627 162.81) (end 227.627 161.6667) (width 0.254) (layer B.Cu) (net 4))
 (segment (start 252.54 172.19) (end 241.11 183.62) (width 0.254) (layer B.Cu) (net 12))
 (segment (start 252.54 167.4603) (end 252.54 172.19) (width 0.254) (layer B.Cu) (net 12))
 (segment (start 276.96 143.0403) (end 252.54 167.4603) (width 0.254) (layer B.Cu) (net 12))
 (segment (start 276.96 141.897) (end 276.96 143.0403) (width 0.254) (layer B.Cu) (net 12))
 (segment (start 238.57 183.62) (end 238.57 181.9318) (width 0.254) (layer B.Cu) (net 11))
 (segment (start 278.1772 140.6798) (end 279.5 139.357) (width 0.254) (layer B.Cu) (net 11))
 (segment (start 276.088 140.6798) (end 278.1772 140.6798) (width 0.254) (layer B.Cu) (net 11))
 (segment (start 250.1512 166.6166) (end 276.088 140.6798) (width 0.254) (layer B.Cu) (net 11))
 (segment (start 250.1512 172.6673) (end 250.1512 166.6166) (width 0.254) (layer B.Cu) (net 11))
 (segment (start 240.8867 181.9318) (end 250.1512 172.6673) (width 0.254) (layer B.Cu) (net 11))
 (segment (start 238.57 181.9318) (end 240.8867 181.9318) (width 0.254) (layer B.Cu) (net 11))
 (segment (start 278.032 180.905) (end 279.627 182.5) (width 0.254) (layer F.Cu) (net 7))
 (segment (start 250.175 180.905) (end 278.032 180.905) (width 0.254) (layer F.Cu) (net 7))
 (segment (start 245.27 176) (end 250.175 180.905) (width 0.254) (layer F.Cu) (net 7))
 (segment (start 226.923 158.8733) (end 227.627 158.8733) (width 0.254) (layer B.Cu) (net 2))
 (segment (start 224.8358 160.9605) (end 226.923 158.8733) (width 0.254) (layer B.Cu) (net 2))
 (segment (start 224.8358 180.8976) (end 224.8358 160.9605) (width 0.254) (layer B.Cu) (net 2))
 (segment (start 225.87 181.9318) (end 224.8358 180.8976) (width 0.254) (layer B.Cu) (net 2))
 (segment (start 225.87 183.62) (end 225.87 181.9318) (width 0.254) (layer B.Cu) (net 2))
 (segment (start 227.627 157.73) (end 227.627 158.8733) (width 0.254) (layer B.Cu) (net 2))
 (segment (start 225.9931 161.6499) (end 227.373 160.27) (width 0.254) (layer B.Cu) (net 3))
 (segment (start 225.9931 163.3449) (end 225.9931 161.6499) (width 0.254) (layer B.Cu) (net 3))
 (segment (start 227.3759 164.7277) (end 225.9931 163.3449) (width 0.254) (layer B.Cu) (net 3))
 (segment (start 227.3759 180.8977) (end 227.3759 164.7277) (width 0.254) (layer B.Cu) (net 3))
 (segment (start 228.41 181.9318) (end 227.3759 180.8977) (width 0.254) (layer B.Cu) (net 3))
 (segment (start 228.41 183.62) (end 228.41 181.9318) (width 0.254) (layer B.Cu) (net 3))
 (segment (start 274.13 168.38) (end 274.13 166.6918) (width 0.254) (layer B.Cu) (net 14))
 (segment (start 278.1638 162.658) (end 274.13 166.6918) (width 0.254) (layer B.Cu) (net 14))
 (segment (start 278.1638 147.432) (end 278.1638 162.658) (width 0.254) (layer B.Cu) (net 14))
 (segment (start 282.04 143.5558) (end 278.1638 147.432) (width 0.254) (layer B.Cu) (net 14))
 (segment (start 282.04 141.897) (end 282.04 143.5558) (width 0.254) (layer B.Cu) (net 14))
 (segment (start 272 172.1982) (end 272 174.2) (width 0.254) (layer F.Cu) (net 14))
 (segment (start 274.13 170.0682) (end 272 172.1982) (width 0.254) (layer F.Cu) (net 14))
 (segment (start 274.13 168.38) (end 274.13 170.0682) (width 0.254) (layer F.Cu) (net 14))
 (segment (start 280.8546 140.7116) (end 282.04 141.897) (width 0.254) (layer B.Cu) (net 14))
 (segment (start 280.8546 139.0613) (end 280.8546 140.7116) (width 0.254) (layer B.Cu) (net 14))
 (segment (start 279.696 137.9027) (end 280.8546 139.0613) (width 0.254) (layer B.Cu) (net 14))
 (segment (start 252.3434 137.9027) (end 279.696 137.9027) (width 0.254) (layer B.Cu) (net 14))
 (segment (start 249.8733 140.3728) (end 252.3434 137.9027) (width 0.254) (layer B.Cu) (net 14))
 (segment (start 249.8733 140.873) (end 249.8733 140.3728) (width 0.254) (layer B.Cu) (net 14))
 (segment (start 248.73 140.873) (end 249.8733 140.873) (width 0.254) (layer B.Cu) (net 14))
 (segment (start 246.19 181.1295) (end 246.19 183.62) (width 0.254) (layer B.Cu) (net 14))
 (segment (start 255.7018 171.6177) (end 246.19 181.1295) (width 0.254) (layer B.Cu) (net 14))
 (segment (start 269.4177 171.6177) (end 255.7018 171.6177) (width 0.254) (layer B.Cu) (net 14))
 (segment (start 272 174.2) (end 269.4177 171.6177) (width 0.254) (layer B.Cu) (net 14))
 (segment (start 242.73 178.4718) (end 242.73 176) (width 0.254) (layer F.Cu) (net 14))
 (segment (start 246.19 181.9318) (end 242.73 178.4718) (width 0.254) (layer F.Cu) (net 14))
 (segment (start 246.19 183.62) (end 246.19 181.9318) (width 0.254) (layer F.Cu) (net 14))
 (segment (start 255.261 170.3208) (end 243.65 181.9318) (width 0.254) (layer B.Cu) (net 13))
 (segment (start 255.261 167.3393) (end 255.261 170.3208) (width 0.254) (layer B.Cu) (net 13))
 (segment (start 273.6552 148.9451) (end 255.261 167.3393) (width 0.254) (layer B.Cu) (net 13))
 (segment (start 275.4414 148.9451) (end 273.6552 148.9451) (width 0.254) (layer B.Cu) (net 13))
 (segment (start 279.5 144.8865) (end 275.4414 148.9451) (width 0.254) (layer B.Cu) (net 13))
 (segment (start 279.5 141.643) (end 279.5 144.8865) (width 0.254) (layer B.Cu) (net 13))
 (segment (start 243.65 183.62) (end 243.65 181.9318) (width 0.254) (layer B.Cu) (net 13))
 (segment (start 271.59 165.5329) (end 271.59 168.38) (width 0.254) (layer F.Cu) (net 17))
 (segment (start 267.0525 160.9954) (end 271.59 165.5329) (width 0.254) (layer F.Cu) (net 17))
 (segment (start 264.2011 160.9954) (end 267.0525 160.9954) (width 0.254) (layer F.Cu) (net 17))
 (segment (start 244.7933 141.5876) (end 264.2011 160.9954) (width 0.254) (layer F.Cu) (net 17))
 (segment (start 244.7933 140.873) (end 244.7933 141.5876) (width 0.254) (layer F.Cu) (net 17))
 (segment (start 243.65 140.873) (end 244.7933 140.873) (width 0.254) (layer F.Cu) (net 17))
 (segment (start 266.6748 166.6918) (end 269.05 166.6918) (width 0.254) (layer F.Cu) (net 18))
 (segment (start 242.2533 142.2703) (end 266.6748 166.6918) (width 0.254) (layer F.Cu) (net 18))
 (segment (start 242.2533 141.127) (end 242.2533 142.2703) (width 0.254) (layer F.Cu) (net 18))
 (segment (start 241.11 141.127) (end 242.2533 141.127) (width 0.254) (layer F.Cu) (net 18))
 (segment (start 269.05 168.38) (end 269.05 166.6918) (width 0.254) (layer F.Cu) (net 18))
 (segment (start 256.5 181.7818) (end 256.5 178.54) (width 0.254) (layer B.Cu) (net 6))
 (segment (start 256.35 181.9318) (end 256.5 181.7818) (width 0.254) (layer B.Cu) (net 6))
 (segment (start 256.35 183.62) (end 256.35 181.9318) (width 0.254) (layer B.Cu) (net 6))
 (segment (start 253.81 176.15) (end 256.5 173.46) (width 0.254) (layer B.Cu) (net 5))
 (segment (start 253.81 183.62) (end 253.81 176.15) (width 0.254) (layer B.Cu) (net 5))
 (segment (start 279.3407 177.1337) (end 279.627 177.42) (width 0.254) (layer B.Cu) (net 9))
 (segment (start 263.6881 177.1337) (end 279.3407 177.1337) (width 0.254) (layer B.Cu) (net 9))
 (segment (start 258.89 181.9318) (end 263.6881 177.1337) (width 0.254) (layer B.Cu) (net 9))
 (segment (start 258.89 183.62) (end 258.89 181.9318) (width 0.254) (layer B.Cu) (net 9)))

